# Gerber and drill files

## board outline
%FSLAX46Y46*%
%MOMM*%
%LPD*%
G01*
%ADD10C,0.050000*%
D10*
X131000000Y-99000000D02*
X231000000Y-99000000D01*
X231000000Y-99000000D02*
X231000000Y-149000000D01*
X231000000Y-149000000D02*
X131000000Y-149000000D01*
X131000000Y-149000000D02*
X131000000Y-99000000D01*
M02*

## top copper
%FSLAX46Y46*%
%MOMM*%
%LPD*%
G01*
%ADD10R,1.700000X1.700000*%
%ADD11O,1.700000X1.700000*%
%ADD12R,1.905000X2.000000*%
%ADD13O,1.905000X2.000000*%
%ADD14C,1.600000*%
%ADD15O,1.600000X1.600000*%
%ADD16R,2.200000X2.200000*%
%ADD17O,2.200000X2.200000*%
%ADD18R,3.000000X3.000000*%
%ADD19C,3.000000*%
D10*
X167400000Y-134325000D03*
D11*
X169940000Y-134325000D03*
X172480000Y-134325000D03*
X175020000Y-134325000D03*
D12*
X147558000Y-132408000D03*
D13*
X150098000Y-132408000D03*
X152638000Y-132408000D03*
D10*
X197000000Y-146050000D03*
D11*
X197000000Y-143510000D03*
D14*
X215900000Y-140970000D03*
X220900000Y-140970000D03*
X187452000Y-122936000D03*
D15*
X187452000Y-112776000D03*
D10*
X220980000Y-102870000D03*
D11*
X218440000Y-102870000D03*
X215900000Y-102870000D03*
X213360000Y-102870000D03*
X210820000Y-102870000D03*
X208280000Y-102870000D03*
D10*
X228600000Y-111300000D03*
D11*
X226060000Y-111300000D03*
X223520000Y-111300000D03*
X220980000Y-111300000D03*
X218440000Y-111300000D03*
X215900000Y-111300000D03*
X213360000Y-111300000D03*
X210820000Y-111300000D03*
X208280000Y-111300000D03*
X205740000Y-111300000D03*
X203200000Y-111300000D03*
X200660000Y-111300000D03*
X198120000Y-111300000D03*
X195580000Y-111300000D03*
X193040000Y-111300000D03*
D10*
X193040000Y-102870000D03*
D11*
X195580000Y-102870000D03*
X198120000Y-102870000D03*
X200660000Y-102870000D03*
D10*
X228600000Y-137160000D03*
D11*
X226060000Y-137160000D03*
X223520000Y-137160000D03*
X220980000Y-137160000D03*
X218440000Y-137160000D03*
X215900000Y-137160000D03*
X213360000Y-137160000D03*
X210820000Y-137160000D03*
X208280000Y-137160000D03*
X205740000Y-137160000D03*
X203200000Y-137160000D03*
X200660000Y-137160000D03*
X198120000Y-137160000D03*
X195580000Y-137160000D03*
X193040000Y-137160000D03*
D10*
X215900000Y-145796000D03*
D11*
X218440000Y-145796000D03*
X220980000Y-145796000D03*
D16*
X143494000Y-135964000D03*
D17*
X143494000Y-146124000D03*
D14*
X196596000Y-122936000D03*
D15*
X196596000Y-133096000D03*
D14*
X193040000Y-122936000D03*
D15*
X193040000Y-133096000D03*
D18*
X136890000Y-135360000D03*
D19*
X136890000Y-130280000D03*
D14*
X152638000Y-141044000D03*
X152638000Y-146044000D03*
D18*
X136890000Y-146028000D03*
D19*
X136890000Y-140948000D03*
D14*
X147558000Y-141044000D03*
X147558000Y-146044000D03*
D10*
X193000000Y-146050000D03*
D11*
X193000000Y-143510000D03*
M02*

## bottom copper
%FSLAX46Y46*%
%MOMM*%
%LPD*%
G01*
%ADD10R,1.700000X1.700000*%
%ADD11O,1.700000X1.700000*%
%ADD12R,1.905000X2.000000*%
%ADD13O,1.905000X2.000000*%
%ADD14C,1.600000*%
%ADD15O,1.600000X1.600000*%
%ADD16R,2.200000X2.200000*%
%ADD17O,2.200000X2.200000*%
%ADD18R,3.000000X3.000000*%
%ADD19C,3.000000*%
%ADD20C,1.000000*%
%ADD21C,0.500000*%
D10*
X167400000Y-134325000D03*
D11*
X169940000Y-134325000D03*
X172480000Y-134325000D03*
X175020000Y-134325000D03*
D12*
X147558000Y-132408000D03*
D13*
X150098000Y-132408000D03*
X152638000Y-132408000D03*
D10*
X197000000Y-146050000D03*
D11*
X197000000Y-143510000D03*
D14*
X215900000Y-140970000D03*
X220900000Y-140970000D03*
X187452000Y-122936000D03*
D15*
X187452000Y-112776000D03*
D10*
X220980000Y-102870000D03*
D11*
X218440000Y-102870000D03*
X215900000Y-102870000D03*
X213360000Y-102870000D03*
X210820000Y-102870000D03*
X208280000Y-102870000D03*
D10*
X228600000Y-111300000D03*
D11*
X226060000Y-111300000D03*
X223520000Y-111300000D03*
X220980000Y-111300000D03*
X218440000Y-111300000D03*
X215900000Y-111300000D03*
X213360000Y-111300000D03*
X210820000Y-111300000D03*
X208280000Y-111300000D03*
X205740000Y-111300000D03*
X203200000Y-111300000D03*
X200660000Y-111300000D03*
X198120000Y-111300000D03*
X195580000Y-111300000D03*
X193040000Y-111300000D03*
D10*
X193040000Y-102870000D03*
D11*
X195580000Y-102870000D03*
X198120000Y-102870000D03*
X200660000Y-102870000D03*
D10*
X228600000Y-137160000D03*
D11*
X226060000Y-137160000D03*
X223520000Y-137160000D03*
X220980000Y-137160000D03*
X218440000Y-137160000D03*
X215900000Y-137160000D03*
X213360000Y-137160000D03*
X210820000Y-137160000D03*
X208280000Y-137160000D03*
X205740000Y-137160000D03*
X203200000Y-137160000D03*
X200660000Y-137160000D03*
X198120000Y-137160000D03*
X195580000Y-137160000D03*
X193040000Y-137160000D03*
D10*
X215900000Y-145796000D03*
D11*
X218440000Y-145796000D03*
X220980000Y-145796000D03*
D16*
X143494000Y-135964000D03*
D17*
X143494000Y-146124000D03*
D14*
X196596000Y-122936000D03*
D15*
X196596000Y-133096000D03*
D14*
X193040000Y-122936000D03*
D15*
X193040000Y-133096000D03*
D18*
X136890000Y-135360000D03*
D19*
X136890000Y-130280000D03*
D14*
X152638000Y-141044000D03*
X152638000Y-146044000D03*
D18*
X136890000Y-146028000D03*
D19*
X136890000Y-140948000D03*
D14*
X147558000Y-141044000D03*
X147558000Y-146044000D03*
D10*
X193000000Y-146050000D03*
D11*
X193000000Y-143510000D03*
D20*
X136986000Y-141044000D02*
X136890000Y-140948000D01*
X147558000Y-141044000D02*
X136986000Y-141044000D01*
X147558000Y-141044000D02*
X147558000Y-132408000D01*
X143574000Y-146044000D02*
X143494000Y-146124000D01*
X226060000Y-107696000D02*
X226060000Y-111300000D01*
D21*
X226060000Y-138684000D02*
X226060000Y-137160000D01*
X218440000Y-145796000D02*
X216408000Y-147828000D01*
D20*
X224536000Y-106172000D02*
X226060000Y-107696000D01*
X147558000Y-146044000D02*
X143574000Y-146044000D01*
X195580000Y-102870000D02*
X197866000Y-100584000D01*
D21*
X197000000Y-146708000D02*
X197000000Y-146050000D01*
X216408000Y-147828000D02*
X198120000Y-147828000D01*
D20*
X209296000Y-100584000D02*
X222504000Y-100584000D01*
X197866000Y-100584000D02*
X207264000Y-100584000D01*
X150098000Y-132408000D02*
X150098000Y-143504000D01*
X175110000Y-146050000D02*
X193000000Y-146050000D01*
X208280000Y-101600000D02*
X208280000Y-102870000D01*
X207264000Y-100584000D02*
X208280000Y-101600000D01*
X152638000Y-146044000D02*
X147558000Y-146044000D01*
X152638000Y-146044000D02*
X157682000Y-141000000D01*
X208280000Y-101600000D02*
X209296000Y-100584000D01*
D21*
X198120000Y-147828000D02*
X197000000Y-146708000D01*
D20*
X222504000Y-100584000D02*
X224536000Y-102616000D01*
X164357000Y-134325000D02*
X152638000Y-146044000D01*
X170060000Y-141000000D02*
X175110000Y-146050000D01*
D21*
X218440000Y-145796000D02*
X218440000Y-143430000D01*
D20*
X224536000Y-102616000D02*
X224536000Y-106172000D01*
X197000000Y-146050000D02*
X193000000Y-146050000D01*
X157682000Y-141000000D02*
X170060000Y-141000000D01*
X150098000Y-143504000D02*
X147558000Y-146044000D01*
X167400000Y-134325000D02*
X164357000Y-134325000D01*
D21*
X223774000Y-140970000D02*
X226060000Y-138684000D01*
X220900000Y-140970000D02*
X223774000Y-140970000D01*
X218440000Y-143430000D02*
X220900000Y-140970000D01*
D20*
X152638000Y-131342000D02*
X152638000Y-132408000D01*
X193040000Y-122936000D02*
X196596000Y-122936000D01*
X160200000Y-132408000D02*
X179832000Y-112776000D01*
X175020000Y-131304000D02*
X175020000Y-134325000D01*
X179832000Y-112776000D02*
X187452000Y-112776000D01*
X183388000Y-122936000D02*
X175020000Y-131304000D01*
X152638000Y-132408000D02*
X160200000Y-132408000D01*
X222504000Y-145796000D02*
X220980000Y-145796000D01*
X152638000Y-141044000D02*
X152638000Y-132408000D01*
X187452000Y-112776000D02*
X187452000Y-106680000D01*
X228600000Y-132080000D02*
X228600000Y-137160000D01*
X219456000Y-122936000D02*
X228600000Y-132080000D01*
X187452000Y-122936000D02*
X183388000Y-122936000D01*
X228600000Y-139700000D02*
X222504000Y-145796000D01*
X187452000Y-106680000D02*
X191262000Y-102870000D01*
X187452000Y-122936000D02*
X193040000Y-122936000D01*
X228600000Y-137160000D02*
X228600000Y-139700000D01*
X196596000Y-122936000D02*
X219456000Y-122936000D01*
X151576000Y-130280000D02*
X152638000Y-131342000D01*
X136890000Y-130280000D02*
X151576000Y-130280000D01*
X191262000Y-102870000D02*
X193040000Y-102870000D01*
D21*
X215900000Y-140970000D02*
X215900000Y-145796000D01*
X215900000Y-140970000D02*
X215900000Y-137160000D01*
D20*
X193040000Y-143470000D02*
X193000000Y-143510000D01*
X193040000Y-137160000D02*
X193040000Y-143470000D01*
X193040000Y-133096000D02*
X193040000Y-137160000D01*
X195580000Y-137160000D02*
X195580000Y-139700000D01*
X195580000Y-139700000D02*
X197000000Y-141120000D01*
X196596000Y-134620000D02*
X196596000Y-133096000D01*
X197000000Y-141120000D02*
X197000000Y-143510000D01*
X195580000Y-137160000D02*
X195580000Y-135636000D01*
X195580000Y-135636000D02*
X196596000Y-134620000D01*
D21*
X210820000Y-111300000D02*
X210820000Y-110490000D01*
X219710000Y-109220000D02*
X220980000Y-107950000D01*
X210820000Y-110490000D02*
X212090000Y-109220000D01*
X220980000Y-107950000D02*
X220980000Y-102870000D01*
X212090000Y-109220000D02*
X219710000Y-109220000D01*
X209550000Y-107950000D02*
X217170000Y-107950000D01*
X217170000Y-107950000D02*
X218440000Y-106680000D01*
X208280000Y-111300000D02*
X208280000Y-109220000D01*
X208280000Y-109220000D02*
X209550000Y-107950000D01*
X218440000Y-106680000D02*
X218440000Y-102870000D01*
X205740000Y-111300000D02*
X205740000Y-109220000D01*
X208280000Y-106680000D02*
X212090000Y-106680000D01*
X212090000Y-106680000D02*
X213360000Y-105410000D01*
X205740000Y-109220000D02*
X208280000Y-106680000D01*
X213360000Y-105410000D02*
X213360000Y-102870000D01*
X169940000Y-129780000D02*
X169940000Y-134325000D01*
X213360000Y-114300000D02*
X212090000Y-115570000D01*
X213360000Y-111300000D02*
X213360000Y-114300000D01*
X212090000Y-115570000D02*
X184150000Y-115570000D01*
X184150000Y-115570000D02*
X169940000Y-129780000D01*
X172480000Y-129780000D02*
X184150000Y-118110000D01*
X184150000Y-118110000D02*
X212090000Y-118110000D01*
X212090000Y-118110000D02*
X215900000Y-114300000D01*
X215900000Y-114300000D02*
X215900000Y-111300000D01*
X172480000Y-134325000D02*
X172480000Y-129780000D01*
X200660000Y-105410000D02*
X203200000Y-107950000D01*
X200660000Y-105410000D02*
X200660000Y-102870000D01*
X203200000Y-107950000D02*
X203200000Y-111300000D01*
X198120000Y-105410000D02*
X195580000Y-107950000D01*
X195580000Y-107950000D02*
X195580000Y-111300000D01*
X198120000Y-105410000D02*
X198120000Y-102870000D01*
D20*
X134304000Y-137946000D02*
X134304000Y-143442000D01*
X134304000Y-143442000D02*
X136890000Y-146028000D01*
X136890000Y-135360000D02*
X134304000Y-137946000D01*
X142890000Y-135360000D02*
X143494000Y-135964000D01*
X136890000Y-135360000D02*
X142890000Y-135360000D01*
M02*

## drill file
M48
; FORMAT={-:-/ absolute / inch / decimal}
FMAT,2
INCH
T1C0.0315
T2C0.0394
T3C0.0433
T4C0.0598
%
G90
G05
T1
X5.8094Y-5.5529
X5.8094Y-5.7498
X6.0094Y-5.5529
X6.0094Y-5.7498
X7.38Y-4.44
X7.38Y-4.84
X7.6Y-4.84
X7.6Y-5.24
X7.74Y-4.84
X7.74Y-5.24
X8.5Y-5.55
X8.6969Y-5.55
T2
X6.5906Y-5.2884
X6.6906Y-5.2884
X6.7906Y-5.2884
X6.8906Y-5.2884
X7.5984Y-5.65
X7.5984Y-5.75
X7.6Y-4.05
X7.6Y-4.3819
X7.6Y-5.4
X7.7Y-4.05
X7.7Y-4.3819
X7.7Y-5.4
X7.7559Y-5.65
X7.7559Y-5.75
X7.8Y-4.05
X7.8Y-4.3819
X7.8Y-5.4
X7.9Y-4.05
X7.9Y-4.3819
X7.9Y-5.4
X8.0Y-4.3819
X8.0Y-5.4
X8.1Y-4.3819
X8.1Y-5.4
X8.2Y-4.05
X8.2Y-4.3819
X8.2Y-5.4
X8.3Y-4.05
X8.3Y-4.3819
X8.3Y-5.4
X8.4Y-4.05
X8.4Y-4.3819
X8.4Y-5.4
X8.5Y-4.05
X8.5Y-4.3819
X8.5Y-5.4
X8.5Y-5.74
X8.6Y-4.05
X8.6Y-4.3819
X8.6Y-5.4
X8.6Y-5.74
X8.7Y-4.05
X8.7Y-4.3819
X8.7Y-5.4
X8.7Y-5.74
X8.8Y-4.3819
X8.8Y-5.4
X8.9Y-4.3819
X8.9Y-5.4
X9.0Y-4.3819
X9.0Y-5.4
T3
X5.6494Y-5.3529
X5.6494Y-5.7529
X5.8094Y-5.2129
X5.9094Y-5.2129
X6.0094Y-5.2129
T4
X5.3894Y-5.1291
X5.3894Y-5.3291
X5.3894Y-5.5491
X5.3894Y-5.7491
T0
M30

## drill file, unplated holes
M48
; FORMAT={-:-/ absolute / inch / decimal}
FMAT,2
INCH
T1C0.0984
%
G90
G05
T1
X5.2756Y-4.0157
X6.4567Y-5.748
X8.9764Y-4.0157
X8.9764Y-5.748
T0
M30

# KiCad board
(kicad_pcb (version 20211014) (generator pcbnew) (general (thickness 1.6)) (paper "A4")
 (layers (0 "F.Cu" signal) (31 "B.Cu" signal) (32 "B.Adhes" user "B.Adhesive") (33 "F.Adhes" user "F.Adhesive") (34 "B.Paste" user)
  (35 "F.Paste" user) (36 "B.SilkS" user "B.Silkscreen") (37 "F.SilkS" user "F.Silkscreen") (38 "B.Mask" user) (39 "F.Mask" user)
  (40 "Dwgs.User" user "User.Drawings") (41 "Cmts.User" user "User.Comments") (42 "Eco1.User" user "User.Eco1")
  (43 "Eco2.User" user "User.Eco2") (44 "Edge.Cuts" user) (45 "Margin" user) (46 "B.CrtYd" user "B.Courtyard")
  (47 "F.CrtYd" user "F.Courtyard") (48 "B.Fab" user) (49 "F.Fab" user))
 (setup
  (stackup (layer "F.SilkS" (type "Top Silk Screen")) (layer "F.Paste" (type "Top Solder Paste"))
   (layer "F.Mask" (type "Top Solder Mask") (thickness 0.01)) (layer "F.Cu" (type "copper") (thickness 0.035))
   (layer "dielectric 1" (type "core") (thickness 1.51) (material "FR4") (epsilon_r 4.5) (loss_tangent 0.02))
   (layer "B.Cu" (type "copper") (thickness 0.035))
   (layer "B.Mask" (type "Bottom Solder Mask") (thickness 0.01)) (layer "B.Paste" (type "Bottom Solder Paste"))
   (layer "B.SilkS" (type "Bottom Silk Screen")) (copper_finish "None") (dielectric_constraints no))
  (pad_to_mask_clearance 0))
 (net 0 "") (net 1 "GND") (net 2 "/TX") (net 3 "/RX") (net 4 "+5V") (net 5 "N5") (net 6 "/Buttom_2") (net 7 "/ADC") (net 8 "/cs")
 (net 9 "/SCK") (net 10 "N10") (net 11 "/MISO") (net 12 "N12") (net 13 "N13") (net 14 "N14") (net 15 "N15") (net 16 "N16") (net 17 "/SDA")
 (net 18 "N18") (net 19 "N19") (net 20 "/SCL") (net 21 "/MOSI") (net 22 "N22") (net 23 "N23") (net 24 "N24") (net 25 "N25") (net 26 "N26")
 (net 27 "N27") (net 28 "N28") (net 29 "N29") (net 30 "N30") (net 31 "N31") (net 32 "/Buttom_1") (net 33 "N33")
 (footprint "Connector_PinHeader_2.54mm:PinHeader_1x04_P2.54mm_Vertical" (layer "F.Cu") (at 167.4 134.325 90)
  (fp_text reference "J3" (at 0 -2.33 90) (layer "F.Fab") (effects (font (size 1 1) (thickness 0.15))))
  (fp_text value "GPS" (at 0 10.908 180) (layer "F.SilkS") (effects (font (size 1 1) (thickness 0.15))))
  (pad "1" thru_hole rect (at 0 0 90) (size 1.7 1.7) (drill 1) (layers *.Cu *.Mask) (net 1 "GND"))
  (pad "2" thru_hole oval (at 0 2.54 90) (size 1.7 1.7) (drill 1) (layers *.Cu *.Mask) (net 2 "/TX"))
  (pad "3" thru_hole oval (at 0 5.08 90) (size 1.7 1.7) (drill 1) (layers *.Cu *.Mask) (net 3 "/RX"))
  (pad "4" thru_hole oval (at 0 7.62 90) (size 1.7 1.7) (drill 1) (layers *.Cu *.Mask) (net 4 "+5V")))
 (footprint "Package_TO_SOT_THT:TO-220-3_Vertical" (layer "F.Cu") (at 147.558 132.408)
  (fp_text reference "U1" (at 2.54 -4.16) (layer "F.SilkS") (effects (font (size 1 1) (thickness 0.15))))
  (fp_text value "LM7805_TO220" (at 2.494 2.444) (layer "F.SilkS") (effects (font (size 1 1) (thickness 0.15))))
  (pad "1" thru_hole rect (at 0 0) (size 1.905 2) (drill 1.1) (layers *.Cu *.Mask) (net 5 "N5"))
  (pad "2" thru_hole oval (at 2.54 0) (size 1.905 2) (drill 1.1) (layers *.Cu *.Mask) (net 1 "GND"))
  (pad "3" thru_hole oval (at 5.08 0) (size 1.905 2) (drill 1.1) (layers *.Cu *.Mask) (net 4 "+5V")))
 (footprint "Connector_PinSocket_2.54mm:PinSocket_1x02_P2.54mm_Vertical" (layer "F.Cu") (at 197 146.05 180)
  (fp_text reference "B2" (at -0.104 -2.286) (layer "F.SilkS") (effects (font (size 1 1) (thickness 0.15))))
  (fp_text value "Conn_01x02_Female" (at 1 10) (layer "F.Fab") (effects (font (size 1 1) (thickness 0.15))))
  (pad "1" thru_hole rect (at 0 0 180) (size 1.7 1.7) (drill 1) (layers *.Cu *.Mask) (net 1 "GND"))
  (pad "2" thru_hole oval (at 0 2.54 180) (size 1.7 1.7) (drill 1) (layers *.Cu *.Mask) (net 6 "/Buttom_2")))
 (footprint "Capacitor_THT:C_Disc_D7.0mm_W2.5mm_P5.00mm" (layer "F.Cu") (at 215.9 140.97)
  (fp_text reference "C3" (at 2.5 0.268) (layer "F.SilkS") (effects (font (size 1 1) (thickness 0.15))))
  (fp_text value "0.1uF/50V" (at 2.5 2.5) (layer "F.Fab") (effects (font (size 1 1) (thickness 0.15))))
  (pad "1" thru_hole circle (at 0 0) (size 1.6 1.6) (drill 0.8) (layers *.Cu *.Mask) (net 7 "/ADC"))
  (pad "2" thru_hole circle (at 5 0) (size 1.6 1.6) (drill 0.8) (layers *.Cu *.Mask) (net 1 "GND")))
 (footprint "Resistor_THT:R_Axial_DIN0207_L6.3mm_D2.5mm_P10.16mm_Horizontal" (layer "F.Cu") (at 187.452 122.936 90)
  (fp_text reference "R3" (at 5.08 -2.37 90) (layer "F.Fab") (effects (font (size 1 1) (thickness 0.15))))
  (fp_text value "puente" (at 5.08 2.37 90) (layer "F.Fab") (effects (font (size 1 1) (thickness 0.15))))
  (pad "1" thru_hole circle (at 0 0 90) (size 1.6 1.6) (drill 0.8) (layers *.Cu *.Mask) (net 4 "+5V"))
  (pad "2" thru_hole oval (at 10.16 0 90) (size 1.6 1.6) (drill 0.8) (layers *.Cu *.Mask) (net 4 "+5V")))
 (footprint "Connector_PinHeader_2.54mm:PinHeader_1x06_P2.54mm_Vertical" (layer "F.Cu") (at 220.98 102.87 -90)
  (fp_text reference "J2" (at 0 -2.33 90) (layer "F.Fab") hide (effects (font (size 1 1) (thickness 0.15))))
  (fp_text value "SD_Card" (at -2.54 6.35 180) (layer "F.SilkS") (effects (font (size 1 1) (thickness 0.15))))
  (pad "1" thru_hole rect (at 0 0 270) (size 1.7 1.7) (drill 1) (layers *.Cu *.Mask) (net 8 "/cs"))
  (pad "2" thru_hole oval (at 0 2.54 270) (size 1.7 1.7) (drill 1) (layers *.Cu *.Mask) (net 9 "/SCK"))
  (pad "3" thru_hole oval (at 0 5.08 270) (size 1.7 1.7) (drill 1) (layers *.Cu *.Mask) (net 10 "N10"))
  (pad "4" thru_hole oval (at 0 7.62 270) (size 1.7 1.7) (drill 1) (layers *.Cu *.Mask) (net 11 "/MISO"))
  (pad "5" thru_hole oval (at 0 10.16 270) (size 1.7 1.7) (drill 1) (layers *.Cu *.Mask) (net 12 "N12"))
  (pad "6" thru_hole oval (at 0 12.7 270) (size 1.7 1.7) (drill 1) (layers *.Cu *.Mask) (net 1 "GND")))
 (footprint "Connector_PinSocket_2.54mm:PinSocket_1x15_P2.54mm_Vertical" (layer "F.Cu") (at 228.6 111.3 -90)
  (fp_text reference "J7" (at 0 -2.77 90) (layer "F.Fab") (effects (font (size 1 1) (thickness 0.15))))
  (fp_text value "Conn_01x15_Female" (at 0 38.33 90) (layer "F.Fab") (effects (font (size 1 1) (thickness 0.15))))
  (pad "1" thru_hole rect (at 0 0 270) (size 1.7 1.7) (drill 1) (layers *.Cu *.Mask) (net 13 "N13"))
  (pad "2" thru_hole oval (at 0 2.54 270) (size 1.7 1.7) (drill 1) (layers *.Cu *.Mask) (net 1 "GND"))
  (pad "3" thru_hole oval (at 0 5.08 270) (size 1.7 1.7) (drill 1) (layers *.Cu *.Mask) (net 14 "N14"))
  (pad "4" thru_hole oval (at 0 7.62 270) (size 1.7 1.7) (drill 1) (layers *.Cu *.Mask) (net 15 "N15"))
  (pad "5" thru_hole oval (at 0 10.16 270) (size 1.7 1.7) (drill 1) (layers *.Cu *.Mask) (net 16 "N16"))
  (pad "6" thru_hole oval (at 0 12.7 270) (size 1.7 1.7) (drill 1) (layers *.Cu *.Mask) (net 3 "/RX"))
  (pad "7" thru_hole oval (at 0 15.24 270) (size 1.7 1.7) (drill 1) (layers *.Cu *.Mask) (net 2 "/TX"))
  (pad "8" thru_hole oval (at 0 17.78 270) (size 1.7 1.7) (drill 1) (layers *.Cu *.Mask) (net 8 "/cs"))
  (pad "9" thru_hole oval (at 0 20.32 270) (size 1.7 1.7) (drill 1) (layers *.Cu *.Mask) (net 9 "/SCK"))
  (pad "10" thru_hole oval (at 0 22.86 270) (size 1.7 1.7) (drill 1) (layers *.Cu *.Mask) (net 11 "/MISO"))
  (pad "11" thru_hole oval (at 0 25.4 270) (size 1.7 1.7) (drill 1) (layers *.Cu *.Mask) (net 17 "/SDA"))
  (pad "12" thru_hole oval (at 0 27.94 270) (size 1.7 1.7) (drill 1) (layers *.Cu *.Mask) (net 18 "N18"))
  (pad "13" thru_hole oval (at 0 30.48 270) (size 1.7 1.7) (drill 1) (layers *.Cu *.Mask) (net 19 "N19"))
  (pad "14" thru_hole oval (at 0 33.02 270) (size 1.7 1.7) (drill 1) (layers *.Cu *.Mask) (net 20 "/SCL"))
  (pad "15" thru_hole oval (at 0 35.56 270) (size 1.7 1.7) (drill 1) (layers *.Cu *.Mask) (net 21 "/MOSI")))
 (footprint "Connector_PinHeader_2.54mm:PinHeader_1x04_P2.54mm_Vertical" (layer "F.Cu") (at 193.04 102.87 90)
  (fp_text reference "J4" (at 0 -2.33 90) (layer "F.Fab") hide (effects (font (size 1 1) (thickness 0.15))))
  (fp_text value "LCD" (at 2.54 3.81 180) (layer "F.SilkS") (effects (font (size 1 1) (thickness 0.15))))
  (pad "1" thru_hole rect (at 0 0 90) (size 1.7 1.7) (drill 1) (layers *.Cu *.Mask) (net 4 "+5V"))
  (pad "2" thru_hole oval (at 0 2.54 90) (size 1.7 1.7) (drill 1) (layers *.Cu *.Mask) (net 1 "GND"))
  (pad "3" thru_hole oval (at 0 5.08 90) (size 1.7 1.7) (drill 1) (layers *.Cu *.Mask) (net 20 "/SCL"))
  (pad "4" thru_hole oval (at 0 7.62 90) (size 1.7 1.7) (drill 1) (layers *.Cu *.Mask) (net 17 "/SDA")))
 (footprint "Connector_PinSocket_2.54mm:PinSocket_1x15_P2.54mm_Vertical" (layer "F.Cu") (at 228.6 137.16 -90)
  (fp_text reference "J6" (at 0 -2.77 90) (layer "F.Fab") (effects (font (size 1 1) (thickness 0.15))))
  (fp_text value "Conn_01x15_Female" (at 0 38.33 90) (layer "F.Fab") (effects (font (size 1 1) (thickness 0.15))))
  (pad "1" thru_hole rect (at 0 0 270) (size 1.7 1.7) (drill 1) (layers *.Cu *.Mask) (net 4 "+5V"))
  (pad "2" thru_hole oval (at 0 2.54 270) (size 1.7 1.7) (drill 1) (layers *.Cu *.Mask) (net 1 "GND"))
  (pad "3" thru_hole oval (at 0 5.08 270) (size 1.7 1.7) (drill 1) (layers *.Cu *.Mask) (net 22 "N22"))
  (pad "4" thru_hole oval (at 0 7.62 270) (size 1.7 1.7) (drill 1) (layers *.Cu *.Mask) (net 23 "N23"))
  (pad "5" thru_hole oval (at 0 10.16 270) (size 1.7 1.7) (drill 1) (layers *.Cu *.Mask) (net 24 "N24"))
  (pad "6" thru_hole oval (at 0 12.7 270) (size 1.7 1.7) (drill 1) (layers *.Cu *.Mask) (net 7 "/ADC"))
  (pad "7" thru_hole oval (at 0 15.24 270) (size 1.7 1.7) (drill 1) (layers *.Cu *.Mask) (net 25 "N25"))
  (pad "8" thru_hole oval (at 0 17.78 270) (size 1.7 1.7) (drill 1) (layers *.Cu *.Mask) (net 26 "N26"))
  (pad "9" thru_hole oval (at 0 20.32 270) (size 1.7 1.7) (drill 1) (layers *.Cu *.Mask) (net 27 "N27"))
  (pad "10" thru_hole oval (at 0 22.86 270) (size 1.7 1.7) (drill 1) (layers *.Cu *.Mask) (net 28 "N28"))
  (pad "11" thru_hole oval (at 0 25.4 270) (size 1.7 1.7) (drill 1) (layers *.Cu *.Mask) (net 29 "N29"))
  (pad "12" thru_hole oval (at 0 27.94 270) (size 1.7 1.7) (drill 1) (layers *.Cu *.Mask) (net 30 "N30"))
  (pad "13" thru_hole oval (at 0 30.48 270) (size 1.7 1.7) (drill 1) (layers *.Cu *.Mask) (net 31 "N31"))
  (pad "14" thru_hole oval (at 0 33.02 270) (size 1.7 1.7) (drill 1) (layers *.Cu *.Mask) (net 6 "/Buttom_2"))
  (pad "15" thru_hole oval (at 0 35.56 270) (size 1.7 1.7) (drill 1) (layers *.Cu *.Mask) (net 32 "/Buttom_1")))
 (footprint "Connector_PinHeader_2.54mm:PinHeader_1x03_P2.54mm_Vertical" (layer "F.Cu") (at 215.9 145.796 90)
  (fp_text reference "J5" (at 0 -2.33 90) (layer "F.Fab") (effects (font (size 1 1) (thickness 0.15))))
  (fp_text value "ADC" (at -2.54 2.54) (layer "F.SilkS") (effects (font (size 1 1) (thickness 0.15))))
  (pad "1" thru_hole rect (at 0 0 90) (size 1.7 1.7) (drill 1) (layers *.Cu *.Mask) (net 7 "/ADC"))
  (pad "2" thru_hole oval (at 0 2.54 90) (size 1.7 1.7) (drill 1) (layers *.Cu *.Mask) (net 1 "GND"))
  (pad "3" thru_hole oval (at 0 5.08 90) (size 1.7 1.7) (drill 1) (layers *.Cu *.Mask) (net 4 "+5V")))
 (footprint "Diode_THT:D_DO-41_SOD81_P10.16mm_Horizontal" (layer "F.Cu") (at 143.494 135.964 -90)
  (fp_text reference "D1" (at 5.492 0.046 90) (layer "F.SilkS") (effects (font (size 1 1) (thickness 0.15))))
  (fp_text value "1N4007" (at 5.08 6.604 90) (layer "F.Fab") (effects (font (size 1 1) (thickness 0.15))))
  (pad "1" thru_hole rect (at 0 0 270) (size 2.2 2.2) (drill 1.1) (layers *.Cu *.Mask) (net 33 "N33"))
  (pad "2" thru_hole oval (at 10.16 0 270) (size 2.2 2.2) (drill 1.1) (layers *.Cu *.Mask) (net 1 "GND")))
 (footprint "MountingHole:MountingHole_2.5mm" (layer "F.Cu") (at 134 102)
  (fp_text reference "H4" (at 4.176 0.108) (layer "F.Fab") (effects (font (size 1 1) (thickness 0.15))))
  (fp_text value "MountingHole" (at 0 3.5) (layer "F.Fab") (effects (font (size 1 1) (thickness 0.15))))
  (pad "" np_thru_hole circle (at 0 0) (size 2.5 2.5) (drill 2.5) (layers *.Cu *.Mask)))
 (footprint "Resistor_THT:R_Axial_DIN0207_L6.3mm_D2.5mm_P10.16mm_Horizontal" (layer "F.Cu") (at 196.596 122.936 -90)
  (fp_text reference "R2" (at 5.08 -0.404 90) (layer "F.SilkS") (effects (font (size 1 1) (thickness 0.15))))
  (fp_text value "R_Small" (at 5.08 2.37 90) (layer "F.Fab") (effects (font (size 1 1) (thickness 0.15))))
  (pad "1" thru_hole circle (at 0 0 270) (size 1.6 1.6) (drill 0.8) (layers *.Cu *.Mask) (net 4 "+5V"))
  (pad "2" thru_hole oval (at 10.16 0 270) (size 1.6 1.6) (drill 0.8) (layers *.Cu *.Mask) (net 6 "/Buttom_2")))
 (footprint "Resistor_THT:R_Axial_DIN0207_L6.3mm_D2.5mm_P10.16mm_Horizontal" (layer "F.Cu") (at 193.04 122.936 -90)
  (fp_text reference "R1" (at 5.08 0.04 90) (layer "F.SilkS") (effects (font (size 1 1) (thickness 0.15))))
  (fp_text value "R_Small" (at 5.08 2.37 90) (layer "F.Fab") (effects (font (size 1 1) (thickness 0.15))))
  (pad "1" thru_hole circle (at 0 0 270) (size 1.6 1.6) (drill 0.8) (layers *.Cu *.Mask) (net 4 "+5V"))
  (pad "2" thru_hole oval (at 10.16 0 270) (size 1.6 1.6) (drill 0.8) (layers *.Cu *.Mask) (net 32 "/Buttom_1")))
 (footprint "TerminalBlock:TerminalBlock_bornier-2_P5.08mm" (layer "F.Cu") (at 136.89 135.36 90)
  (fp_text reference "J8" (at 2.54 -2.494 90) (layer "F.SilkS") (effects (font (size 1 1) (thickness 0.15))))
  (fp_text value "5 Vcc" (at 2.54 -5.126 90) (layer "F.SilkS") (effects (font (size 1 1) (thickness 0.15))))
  (pad "1" thru_hole rect (at 0 0 90) (size 3 3) (drill 1.52) (layers *.Cu *.Mask) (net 33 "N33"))
  (pad "2" thru_hole circle (at 5.08 0 90) (size 3 3) (drill 1.52) (layers *.Cu *.Mask) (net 4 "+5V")))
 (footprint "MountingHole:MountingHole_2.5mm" (layer "F.Cu") (at 228 102)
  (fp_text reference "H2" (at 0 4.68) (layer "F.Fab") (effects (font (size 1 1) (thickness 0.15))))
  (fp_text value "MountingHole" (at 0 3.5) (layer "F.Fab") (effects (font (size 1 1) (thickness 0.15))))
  (pad "" np_thru_hole circle (at 0 0) (size 2.5 2.5) (drill 2.5) (layers *.Cu *.Mask)))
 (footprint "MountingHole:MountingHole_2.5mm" (layer "F.Cu") (at 228 146)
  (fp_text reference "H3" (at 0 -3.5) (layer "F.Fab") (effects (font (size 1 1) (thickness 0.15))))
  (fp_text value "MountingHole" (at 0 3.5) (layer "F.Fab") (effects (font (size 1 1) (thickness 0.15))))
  (pad "" np_thru_hole circle (at 0 0) (size 2.5 2.5) (drill 2.5) (layers *.Cu *.Mask)))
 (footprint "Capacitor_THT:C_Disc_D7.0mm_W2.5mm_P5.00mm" (layer "F.Cu") (at 152.638 141.044 -90)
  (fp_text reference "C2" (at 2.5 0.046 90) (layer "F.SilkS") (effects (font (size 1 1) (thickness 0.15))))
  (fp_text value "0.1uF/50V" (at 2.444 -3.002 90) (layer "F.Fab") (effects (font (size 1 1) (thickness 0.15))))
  (pad "1" thru_hole circle (at 0 0 270) (size 1.6 1.6) (drill 0.8) (layers *.Cu *.Mask) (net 4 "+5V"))
  (pad "2" thru_hole circle (at 5 0 270) (size 1.6 1.6) (drill 0.8) (layers *.Cu *.Mask) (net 1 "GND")))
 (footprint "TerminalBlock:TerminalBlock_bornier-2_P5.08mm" (layer "F.Cu") (at 136.89 146.028 90)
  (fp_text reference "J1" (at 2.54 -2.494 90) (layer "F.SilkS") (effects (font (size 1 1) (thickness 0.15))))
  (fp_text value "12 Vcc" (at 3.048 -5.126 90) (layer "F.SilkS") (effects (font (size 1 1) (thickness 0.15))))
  (pad "1" thru_hole rect (at 0 0 90) (size 3 3) (drill 1.52) (layers *.Cu *.Mask) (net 33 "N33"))
  (pad "2" thru_hole circle (at 5.08 0 90) (size 3 3) (drill 1.52) (layers *.Cu *.Mask) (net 5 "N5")))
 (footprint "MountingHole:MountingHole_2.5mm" (layer "F.Cu") (at 164 146)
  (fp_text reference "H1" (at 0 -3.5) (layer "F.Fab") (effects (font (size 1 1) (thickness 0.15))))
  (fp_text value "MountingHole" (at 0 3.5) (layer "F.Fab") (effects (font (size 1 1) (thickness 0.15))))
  (pad "" np_thru_hole circle (at 0 0) (size 2.5 2.5) (drill 2.5) (layers *.Cu *.Mask)))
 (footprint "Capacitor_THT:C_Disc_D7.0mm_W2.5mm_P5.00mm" (layer "F.Cu") (at 147.558 141.044 -90)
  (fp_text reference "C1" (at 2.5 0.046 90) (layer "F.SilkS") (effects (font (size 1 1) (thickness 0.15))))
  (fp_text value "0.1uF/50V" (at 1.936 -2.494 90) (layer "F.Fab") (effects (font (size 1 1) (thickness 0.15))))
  (pad "1" thru_hole circle (at 0 0 270) (size 1.6 1.6) (drill 0.8) (layers *.Cu *.Mask) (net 5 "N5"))
  (pad "2" thru_hole circle (at 5 0 270) (size 1.6 1.6) (drill 0.8) (layers *.Cu *.Mask) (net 1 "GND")))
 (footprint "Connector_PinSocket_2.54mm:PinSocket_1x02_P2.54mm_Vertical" (layer "F.Cu") (at 193 146.05 180)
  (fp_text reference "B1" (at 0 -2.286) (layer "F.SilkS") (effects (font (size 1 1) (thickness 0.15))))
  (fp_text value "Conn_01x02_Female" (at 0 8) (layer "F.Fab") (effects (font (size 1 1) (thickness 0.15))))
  (pad "1" thru_hole rect (at 0 0 180) (size 1.7 1.7) (drill 1) (layers *.Cu *.Mask) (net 1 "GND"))
  (pad "2" thru_hole oval (at 0 2.54 180) (size 1.7 1.7) (drill 1) (layers *.Cu *.Mask) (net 32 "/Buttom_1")))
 (gr_rect (start 131 99) (end 231 149) (layer "Edge.Cuts") (width 0.05) (fill none))
 (segment (start 136.986 141.044) (end 136.89 140.948) (width 1) (layer "B.Cu") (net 5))
 (segment (start 147.558 141.044) (end 136.986 141.044) (width 1) (layer "B.Cu") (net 5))
 (segment (start 147.558 141.044) (end 147.558 132.408) (width 1) (layer "B.Cu") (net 5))
 (segment (start 143.574 146.044) (end 143.494 146.124) (width 1) (layer "B.Cu") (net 1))
 (segment (start 226.06 107.696) (end 226.06 111.3) (width 1) (layer "B.Cu") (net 1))
 (segment (start 226.06 138.684) (end 226.06 137.16) (width 0.5) (layer "B.Cu") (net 1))
 (segment (start 218.44 145.796) (end 216.408 147.828) (width 0.5) (layer "B.Cu") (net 1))
 (segment (start 224.536 106.172) (end 226.06 107.696) (width 1) (layer "B.Cu") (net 1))
 (segment (start 147.558 146.044) (end 143.574 146.044) (width 1) (layer "B.Cu") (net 1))
 (segment (start 195.58 102.87) (end 197.866 100.584) (width 1) (layer "B.Cu") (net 1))
 (segment (start 197 146.708) (end 197 146.05) (width 0.5) (layer "B.Cu") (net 1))
 (segment (start 216.408 147.828) (end 198.12 147.828) (width 0.5) (layer "B.Cu") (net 1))
 (segment (start 209.296 100.584) (end 222.504 100.584) (width 1) (layer "B.Cu") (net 1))
 (segment (start 197.866 100.584) (end 207.264 100.584) (width 1) (layer "B.Cu") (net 1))
 (segment (start 150.098 132.408) (end 150.098 143.504) (width 1) (layer "B.Cu") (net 1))
 (segment (start 175.11 146.05) (end 193 146.05) (width 1) (layer "B.Cu") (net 1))
 (segment (start 208.28 101.6) (end 208.28 102.87) (width 1) (layer "B.Cu") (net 1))
 (segment (start 207.264 100.584) (end 208.28 101.6) (width 1) (layer "B.Cu") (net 1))
 (segment (start 152.638 146.044) (end 147.558 146.044) (width 1) (layer "B.Cu") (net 1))
 (segment (start 152.638 146.044) (end 157.682 141) (width 1) (layer "B.Cu") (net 1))
 (segment (start 208.28 101.6) (end 209.296 100.584) (width 1) (layer "B.Cu") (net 1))
 (segment (start 198.12 147.828) (end 197 146.708) (width 0.5) (layer "B.Cu") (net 1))
 (segment (start 222.504 100.584) (end 224.536 102.616) (width 1) (layer "B.Cu") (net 1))
 (segment (start 164.357 134.325) (end 152.638 146.044) (width 1) (layer "B.Cu") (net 1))
 (segment (start 170.06 141) (end 175.11 146.05) (width 1) (layer "B.Cu") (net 1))
 (segment (start 218.44 145.796) (end 218.44 143.43) (width 0.5) (layer "B.Cu") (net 1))
 (segment (start 224.536 102.616) (end 224.536 106.172) (width 1) (layer "B.Cu") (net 1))
 (segment (start 197 146.05) (end 193 146.05) (width 1) (layer "B.Cu") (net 1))
 (segment (start 157.682 141) (end 170.06 141) (width 1) (layer "B.Cu") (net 1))
 (segment (start 150.098 143.504) (end 147.558 146.044) (width 1) (layer "B.Cu") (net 1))
 (segment (start 167.4 134.325) (end 164.357 134.325) (width 1) (layer "B.Cu") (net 1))
 (segment (start 223.774 140.97) (end 226.06 138.684) (width 0.5) (layer "B.Cu") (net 1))
 (segment (start 220.9 140.97) (end 223.774 140.97) (width 0.5) (layer "B.Cu") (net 1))
 (segment (start 218.44 143.43) (end 220.9 140.97) (width 0.5) (layer "B.Cu") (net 1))
 (segment (start 152.638 131.342) (end 152.638 132.408) (width 1) (layer "B.Cu") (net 4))
 (segment (start 193.04 122.936) (end 196.596 122.936) (width 1) (layer "B.Cu") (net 4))
 (segment (start 160.2 132.408) (end 179.832 112.776) (width 1) (layer "B.Cu") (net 4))
 (segment (start 175.02 131.304) (end 175.02 134.325) (width 1) (layer "B.Cu") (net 4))
 (segment (start 179.832 112.776) (end 187.452 112.776) (width 1) (layer "B.Cu") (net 4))
 (segment (start 183.388 122.936) (end 175.02 131.304) (width 1) (layer "B.Cu") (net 4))
 (segment (start 152.638 132.408) (end 160.2 132.408) (width 1) (layer "B.Cu") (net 4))
 (segment (start 222.504 145.796) (end 220.98 145.796) (width 1) (layer "B.Cu") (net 4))
 (segment (start 152.638 141.044) (end 152.638 132.408) (width 1) (layer "B.Cu") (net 4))
 (segment (start 187.452 112.776) (end 187.452 106.68) (width 1) (layer "B.Cu") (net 4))
 (segment (start 228.6 132.08) (end 228.6 137.16) (width 1) (layer "B.Cu") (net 4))
 (segment (start 219.456 122.936) (end 228.6 132.08) (width 1) (layer "B.Cu") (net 4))
 (segment (start 187.452 122.936) (end 183.388 122.936) (width 1) (layer "B.Cu") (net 4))
 (segment (start 228.6 139.7) (end 222.504 145.796) (width 1) (layer "B.Cu") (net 4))
 (segment (start 187.452 106.68) (end 191.262 102.87) (width 1) (layer "B.Cu") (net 4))
 (segment (start 187.452 122.936) (end 193.04 122.936) (width 1) (layer "B.Cu") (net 4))
 (segment (start 228.6 137.16) (end 228.6 139.7) (width 1) (layer "B.Cu") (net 4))
 (segment (start 196.596 122.936) (end 219.456 122.936) (width 1) (layer "B.Cu") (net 4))
 (segment (start 151.576 130.28) (end 152.638 131.342) (width 1) (layer "B.Cu") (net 4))
 (segment (start 136.89 130.28) (end 151.576 130.28) (width 1) (layer "B.Cu") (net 4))
 (segment (start 191.262 102.87) (end 193.04 102.87) (width 1) (layer "B.Cu") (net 4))
 (segment (start 215.9 140.97) (end 215.9 145.796) (width 0.5) (layer "B.Cu") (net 7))
 (segment (start 215.9 140.97) (end 215.9 137.16) (width 0.5) (layer "B.Cu") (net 7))
 (segment (start 193.04 143.47) (end 193 143.51) (width 1) (layer "B.Cu") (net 32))
 (segment (start 193.04 137.16) (end 193.04 143.47) (width 1) (layer "B.Cu") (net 32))
 (segment (start 193.04 133.096) (end 193.04 137.16) (width 1) (layer "B.Cu") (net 32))
 (segment (start 195.58 137.16) (end 195.58 139.7) (width 1) (layer "B.Cu") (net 6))
 (segment (start 195.58 139.7) (end 197 141.12) (width 1) (layer "B.Cu") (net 6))
 (segment (start 196.596 134.62) (end 196.596 133.096) (width 1) (layer "B.Cu") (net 6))
 (segment (start 197 141.12) (end 197 143.51) (width 1) (layer "B.Cu") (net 6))
 (segment (start 195.58 137.16) (end 195.58 135.636) (width 1) (layer "B.Cu") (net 6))
 (segment (start 195.58 135.636) (end 196.596 134.62) (width 1) (layer "B.Cu") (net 6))
 (segment (start 210.82 111.3) (end 210.82 110.49) (width 0.5) (layer "B.Cu") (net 8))
 (segment (start 219.71 109.22) (end 220.98 107.95) (width 0.5) (layer "B.Cu") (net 8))
 (segment (start 210.82 110.49) (end 212.09 109.22) (width 0.5) (layer "B.Cu") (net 8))
 (segment (start 220.98 107.95) (end 220.98 102.87) (width 0.5) (layer "B.Cu") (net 8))
 (segment (start 212.09 109.22) (end 219.71 109.22) (width 0.5) (layer "B.Cu") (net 8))
 (segment (start 209.55 107.95) (end 217.17 107.95) (width 0.5) (layer "B.Cu") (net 9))
 (segment (start 217.17 107.95) (end 218.44 106.68) (width 0.5) (layer "B.Cu") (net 9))
 (segment (start 208.28 111.3) (end 208.28 109.22) (width 0.5) (layer "B.Cu") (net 9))
 (segment (start 208.28 109.22) (end 209.55 107.95) (width 0.5) (layer "B.Cu") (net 9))
 (segment (start 218.44 106.68) (end 218.44 102.87) (width 0.5) (layer "B.Cu") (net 9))
 (segment (start 205.74 111.3) (end 205.74 109.22) (width 0.5) (layer "B.Cu") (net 11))
 (segment (start 208.28 106.68) (end 212.09 106.68) (width 0.5) (layer "B.Cu") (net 11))
 (segment (start 212.09 106.68) (end 213.36 105.41) (width 0.5) (layer "B.Cu") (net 11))
 (segment (start 205.74 109.22) (end 208.28 106.68) (width 0.5) (layer "B.Cu") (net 11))
 (segment (start 213.36 105.41) (end 213.36 102.87) (width 0.5) (layer "B.Cu") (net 11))
 (segment (start 169.94 129.78) (end 169.94 134.325) (width 0.5) (layer "B.Cu") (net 2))
 (segment (start 213.36 114.3) (end 212.09 115.57) (width 0.5) (layer "B.Cu") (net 2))
 (segment (start 213.36 111.3) (end 213.36 114.3) (width 0.5) (layer "B.Cu") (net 2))
 (segment (start 212.09 115.57) (end 184.15 115.57) (width 0.5) (layer "B.Cu") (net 2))
 (segment (start 184.15 115.57) (end 169.94 129.78) (width 0.5) (layer "B.Cu") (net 2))
 (segment (start 172.48 129.78) (end 184.15 118.11) (width 0.5) (layer "B.Cu") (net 3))
 (segment (start 184.15 118.11) (end 212.09 118.11) (width 0.5) (layer "B.Cu") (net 3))
 (segment (start 212.09 118.11) (end 215.9 114.3) (width 0.5) (layer "B.Cu") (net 3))
 (segment (start 215.9 114.3) (end 215.9 111.3) (width 0.5) (layer "B.Cu") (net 3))
 (segment (start 172.48 134.325) (end 172.48 129.78) (width 0.5) (layer "B.Cu") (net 3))
 (segment (start 200.66 105.41) (end 203.2 107.95) (width 0.5) (layer "B.Cu") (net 17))
 (segment (start 200.66 105.41) (end 200.66 102.87) (width 0.5) (layer "B.Cu") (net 17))
 (segment (start 203.2 107.95) (end 203.2 111.3) (width 0.5) (layer "B.Cu") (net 17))
 (segment (start 198.12 105.41) (end 195.58 107.95) (width 0.5) (layer "B.Cu") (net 20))
 (segment (start 195.58 107.95) (end 195.58 111.3) (width 0.5) (layer "B.Cu") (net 20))
 (segment (start 198.12 105.41) (end 198.12 102.87) (width 0.5) (layer "B.Cu") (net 20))
 (segment (start 134.304 137.946) (end 134.304 143.442) (width 1) (layer "B.Cu") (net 33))
 (segment (start 134.304 143.442) (end 136.89 146.028) (width 1) (layer "B.Cu") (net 33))
 (segment (start 136.89 135.36) (end 134.304 137.946) (width 1) (layer "B.Cu") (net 33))
 (segment (start 142.89 135.36) (end 143.494 135.964) (width 1) (layer "B.Cu") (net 33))
 (segment (start 136.89 135.36) (end 142.89 135.36) (width 1) (layer "B.Cu") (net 33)))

